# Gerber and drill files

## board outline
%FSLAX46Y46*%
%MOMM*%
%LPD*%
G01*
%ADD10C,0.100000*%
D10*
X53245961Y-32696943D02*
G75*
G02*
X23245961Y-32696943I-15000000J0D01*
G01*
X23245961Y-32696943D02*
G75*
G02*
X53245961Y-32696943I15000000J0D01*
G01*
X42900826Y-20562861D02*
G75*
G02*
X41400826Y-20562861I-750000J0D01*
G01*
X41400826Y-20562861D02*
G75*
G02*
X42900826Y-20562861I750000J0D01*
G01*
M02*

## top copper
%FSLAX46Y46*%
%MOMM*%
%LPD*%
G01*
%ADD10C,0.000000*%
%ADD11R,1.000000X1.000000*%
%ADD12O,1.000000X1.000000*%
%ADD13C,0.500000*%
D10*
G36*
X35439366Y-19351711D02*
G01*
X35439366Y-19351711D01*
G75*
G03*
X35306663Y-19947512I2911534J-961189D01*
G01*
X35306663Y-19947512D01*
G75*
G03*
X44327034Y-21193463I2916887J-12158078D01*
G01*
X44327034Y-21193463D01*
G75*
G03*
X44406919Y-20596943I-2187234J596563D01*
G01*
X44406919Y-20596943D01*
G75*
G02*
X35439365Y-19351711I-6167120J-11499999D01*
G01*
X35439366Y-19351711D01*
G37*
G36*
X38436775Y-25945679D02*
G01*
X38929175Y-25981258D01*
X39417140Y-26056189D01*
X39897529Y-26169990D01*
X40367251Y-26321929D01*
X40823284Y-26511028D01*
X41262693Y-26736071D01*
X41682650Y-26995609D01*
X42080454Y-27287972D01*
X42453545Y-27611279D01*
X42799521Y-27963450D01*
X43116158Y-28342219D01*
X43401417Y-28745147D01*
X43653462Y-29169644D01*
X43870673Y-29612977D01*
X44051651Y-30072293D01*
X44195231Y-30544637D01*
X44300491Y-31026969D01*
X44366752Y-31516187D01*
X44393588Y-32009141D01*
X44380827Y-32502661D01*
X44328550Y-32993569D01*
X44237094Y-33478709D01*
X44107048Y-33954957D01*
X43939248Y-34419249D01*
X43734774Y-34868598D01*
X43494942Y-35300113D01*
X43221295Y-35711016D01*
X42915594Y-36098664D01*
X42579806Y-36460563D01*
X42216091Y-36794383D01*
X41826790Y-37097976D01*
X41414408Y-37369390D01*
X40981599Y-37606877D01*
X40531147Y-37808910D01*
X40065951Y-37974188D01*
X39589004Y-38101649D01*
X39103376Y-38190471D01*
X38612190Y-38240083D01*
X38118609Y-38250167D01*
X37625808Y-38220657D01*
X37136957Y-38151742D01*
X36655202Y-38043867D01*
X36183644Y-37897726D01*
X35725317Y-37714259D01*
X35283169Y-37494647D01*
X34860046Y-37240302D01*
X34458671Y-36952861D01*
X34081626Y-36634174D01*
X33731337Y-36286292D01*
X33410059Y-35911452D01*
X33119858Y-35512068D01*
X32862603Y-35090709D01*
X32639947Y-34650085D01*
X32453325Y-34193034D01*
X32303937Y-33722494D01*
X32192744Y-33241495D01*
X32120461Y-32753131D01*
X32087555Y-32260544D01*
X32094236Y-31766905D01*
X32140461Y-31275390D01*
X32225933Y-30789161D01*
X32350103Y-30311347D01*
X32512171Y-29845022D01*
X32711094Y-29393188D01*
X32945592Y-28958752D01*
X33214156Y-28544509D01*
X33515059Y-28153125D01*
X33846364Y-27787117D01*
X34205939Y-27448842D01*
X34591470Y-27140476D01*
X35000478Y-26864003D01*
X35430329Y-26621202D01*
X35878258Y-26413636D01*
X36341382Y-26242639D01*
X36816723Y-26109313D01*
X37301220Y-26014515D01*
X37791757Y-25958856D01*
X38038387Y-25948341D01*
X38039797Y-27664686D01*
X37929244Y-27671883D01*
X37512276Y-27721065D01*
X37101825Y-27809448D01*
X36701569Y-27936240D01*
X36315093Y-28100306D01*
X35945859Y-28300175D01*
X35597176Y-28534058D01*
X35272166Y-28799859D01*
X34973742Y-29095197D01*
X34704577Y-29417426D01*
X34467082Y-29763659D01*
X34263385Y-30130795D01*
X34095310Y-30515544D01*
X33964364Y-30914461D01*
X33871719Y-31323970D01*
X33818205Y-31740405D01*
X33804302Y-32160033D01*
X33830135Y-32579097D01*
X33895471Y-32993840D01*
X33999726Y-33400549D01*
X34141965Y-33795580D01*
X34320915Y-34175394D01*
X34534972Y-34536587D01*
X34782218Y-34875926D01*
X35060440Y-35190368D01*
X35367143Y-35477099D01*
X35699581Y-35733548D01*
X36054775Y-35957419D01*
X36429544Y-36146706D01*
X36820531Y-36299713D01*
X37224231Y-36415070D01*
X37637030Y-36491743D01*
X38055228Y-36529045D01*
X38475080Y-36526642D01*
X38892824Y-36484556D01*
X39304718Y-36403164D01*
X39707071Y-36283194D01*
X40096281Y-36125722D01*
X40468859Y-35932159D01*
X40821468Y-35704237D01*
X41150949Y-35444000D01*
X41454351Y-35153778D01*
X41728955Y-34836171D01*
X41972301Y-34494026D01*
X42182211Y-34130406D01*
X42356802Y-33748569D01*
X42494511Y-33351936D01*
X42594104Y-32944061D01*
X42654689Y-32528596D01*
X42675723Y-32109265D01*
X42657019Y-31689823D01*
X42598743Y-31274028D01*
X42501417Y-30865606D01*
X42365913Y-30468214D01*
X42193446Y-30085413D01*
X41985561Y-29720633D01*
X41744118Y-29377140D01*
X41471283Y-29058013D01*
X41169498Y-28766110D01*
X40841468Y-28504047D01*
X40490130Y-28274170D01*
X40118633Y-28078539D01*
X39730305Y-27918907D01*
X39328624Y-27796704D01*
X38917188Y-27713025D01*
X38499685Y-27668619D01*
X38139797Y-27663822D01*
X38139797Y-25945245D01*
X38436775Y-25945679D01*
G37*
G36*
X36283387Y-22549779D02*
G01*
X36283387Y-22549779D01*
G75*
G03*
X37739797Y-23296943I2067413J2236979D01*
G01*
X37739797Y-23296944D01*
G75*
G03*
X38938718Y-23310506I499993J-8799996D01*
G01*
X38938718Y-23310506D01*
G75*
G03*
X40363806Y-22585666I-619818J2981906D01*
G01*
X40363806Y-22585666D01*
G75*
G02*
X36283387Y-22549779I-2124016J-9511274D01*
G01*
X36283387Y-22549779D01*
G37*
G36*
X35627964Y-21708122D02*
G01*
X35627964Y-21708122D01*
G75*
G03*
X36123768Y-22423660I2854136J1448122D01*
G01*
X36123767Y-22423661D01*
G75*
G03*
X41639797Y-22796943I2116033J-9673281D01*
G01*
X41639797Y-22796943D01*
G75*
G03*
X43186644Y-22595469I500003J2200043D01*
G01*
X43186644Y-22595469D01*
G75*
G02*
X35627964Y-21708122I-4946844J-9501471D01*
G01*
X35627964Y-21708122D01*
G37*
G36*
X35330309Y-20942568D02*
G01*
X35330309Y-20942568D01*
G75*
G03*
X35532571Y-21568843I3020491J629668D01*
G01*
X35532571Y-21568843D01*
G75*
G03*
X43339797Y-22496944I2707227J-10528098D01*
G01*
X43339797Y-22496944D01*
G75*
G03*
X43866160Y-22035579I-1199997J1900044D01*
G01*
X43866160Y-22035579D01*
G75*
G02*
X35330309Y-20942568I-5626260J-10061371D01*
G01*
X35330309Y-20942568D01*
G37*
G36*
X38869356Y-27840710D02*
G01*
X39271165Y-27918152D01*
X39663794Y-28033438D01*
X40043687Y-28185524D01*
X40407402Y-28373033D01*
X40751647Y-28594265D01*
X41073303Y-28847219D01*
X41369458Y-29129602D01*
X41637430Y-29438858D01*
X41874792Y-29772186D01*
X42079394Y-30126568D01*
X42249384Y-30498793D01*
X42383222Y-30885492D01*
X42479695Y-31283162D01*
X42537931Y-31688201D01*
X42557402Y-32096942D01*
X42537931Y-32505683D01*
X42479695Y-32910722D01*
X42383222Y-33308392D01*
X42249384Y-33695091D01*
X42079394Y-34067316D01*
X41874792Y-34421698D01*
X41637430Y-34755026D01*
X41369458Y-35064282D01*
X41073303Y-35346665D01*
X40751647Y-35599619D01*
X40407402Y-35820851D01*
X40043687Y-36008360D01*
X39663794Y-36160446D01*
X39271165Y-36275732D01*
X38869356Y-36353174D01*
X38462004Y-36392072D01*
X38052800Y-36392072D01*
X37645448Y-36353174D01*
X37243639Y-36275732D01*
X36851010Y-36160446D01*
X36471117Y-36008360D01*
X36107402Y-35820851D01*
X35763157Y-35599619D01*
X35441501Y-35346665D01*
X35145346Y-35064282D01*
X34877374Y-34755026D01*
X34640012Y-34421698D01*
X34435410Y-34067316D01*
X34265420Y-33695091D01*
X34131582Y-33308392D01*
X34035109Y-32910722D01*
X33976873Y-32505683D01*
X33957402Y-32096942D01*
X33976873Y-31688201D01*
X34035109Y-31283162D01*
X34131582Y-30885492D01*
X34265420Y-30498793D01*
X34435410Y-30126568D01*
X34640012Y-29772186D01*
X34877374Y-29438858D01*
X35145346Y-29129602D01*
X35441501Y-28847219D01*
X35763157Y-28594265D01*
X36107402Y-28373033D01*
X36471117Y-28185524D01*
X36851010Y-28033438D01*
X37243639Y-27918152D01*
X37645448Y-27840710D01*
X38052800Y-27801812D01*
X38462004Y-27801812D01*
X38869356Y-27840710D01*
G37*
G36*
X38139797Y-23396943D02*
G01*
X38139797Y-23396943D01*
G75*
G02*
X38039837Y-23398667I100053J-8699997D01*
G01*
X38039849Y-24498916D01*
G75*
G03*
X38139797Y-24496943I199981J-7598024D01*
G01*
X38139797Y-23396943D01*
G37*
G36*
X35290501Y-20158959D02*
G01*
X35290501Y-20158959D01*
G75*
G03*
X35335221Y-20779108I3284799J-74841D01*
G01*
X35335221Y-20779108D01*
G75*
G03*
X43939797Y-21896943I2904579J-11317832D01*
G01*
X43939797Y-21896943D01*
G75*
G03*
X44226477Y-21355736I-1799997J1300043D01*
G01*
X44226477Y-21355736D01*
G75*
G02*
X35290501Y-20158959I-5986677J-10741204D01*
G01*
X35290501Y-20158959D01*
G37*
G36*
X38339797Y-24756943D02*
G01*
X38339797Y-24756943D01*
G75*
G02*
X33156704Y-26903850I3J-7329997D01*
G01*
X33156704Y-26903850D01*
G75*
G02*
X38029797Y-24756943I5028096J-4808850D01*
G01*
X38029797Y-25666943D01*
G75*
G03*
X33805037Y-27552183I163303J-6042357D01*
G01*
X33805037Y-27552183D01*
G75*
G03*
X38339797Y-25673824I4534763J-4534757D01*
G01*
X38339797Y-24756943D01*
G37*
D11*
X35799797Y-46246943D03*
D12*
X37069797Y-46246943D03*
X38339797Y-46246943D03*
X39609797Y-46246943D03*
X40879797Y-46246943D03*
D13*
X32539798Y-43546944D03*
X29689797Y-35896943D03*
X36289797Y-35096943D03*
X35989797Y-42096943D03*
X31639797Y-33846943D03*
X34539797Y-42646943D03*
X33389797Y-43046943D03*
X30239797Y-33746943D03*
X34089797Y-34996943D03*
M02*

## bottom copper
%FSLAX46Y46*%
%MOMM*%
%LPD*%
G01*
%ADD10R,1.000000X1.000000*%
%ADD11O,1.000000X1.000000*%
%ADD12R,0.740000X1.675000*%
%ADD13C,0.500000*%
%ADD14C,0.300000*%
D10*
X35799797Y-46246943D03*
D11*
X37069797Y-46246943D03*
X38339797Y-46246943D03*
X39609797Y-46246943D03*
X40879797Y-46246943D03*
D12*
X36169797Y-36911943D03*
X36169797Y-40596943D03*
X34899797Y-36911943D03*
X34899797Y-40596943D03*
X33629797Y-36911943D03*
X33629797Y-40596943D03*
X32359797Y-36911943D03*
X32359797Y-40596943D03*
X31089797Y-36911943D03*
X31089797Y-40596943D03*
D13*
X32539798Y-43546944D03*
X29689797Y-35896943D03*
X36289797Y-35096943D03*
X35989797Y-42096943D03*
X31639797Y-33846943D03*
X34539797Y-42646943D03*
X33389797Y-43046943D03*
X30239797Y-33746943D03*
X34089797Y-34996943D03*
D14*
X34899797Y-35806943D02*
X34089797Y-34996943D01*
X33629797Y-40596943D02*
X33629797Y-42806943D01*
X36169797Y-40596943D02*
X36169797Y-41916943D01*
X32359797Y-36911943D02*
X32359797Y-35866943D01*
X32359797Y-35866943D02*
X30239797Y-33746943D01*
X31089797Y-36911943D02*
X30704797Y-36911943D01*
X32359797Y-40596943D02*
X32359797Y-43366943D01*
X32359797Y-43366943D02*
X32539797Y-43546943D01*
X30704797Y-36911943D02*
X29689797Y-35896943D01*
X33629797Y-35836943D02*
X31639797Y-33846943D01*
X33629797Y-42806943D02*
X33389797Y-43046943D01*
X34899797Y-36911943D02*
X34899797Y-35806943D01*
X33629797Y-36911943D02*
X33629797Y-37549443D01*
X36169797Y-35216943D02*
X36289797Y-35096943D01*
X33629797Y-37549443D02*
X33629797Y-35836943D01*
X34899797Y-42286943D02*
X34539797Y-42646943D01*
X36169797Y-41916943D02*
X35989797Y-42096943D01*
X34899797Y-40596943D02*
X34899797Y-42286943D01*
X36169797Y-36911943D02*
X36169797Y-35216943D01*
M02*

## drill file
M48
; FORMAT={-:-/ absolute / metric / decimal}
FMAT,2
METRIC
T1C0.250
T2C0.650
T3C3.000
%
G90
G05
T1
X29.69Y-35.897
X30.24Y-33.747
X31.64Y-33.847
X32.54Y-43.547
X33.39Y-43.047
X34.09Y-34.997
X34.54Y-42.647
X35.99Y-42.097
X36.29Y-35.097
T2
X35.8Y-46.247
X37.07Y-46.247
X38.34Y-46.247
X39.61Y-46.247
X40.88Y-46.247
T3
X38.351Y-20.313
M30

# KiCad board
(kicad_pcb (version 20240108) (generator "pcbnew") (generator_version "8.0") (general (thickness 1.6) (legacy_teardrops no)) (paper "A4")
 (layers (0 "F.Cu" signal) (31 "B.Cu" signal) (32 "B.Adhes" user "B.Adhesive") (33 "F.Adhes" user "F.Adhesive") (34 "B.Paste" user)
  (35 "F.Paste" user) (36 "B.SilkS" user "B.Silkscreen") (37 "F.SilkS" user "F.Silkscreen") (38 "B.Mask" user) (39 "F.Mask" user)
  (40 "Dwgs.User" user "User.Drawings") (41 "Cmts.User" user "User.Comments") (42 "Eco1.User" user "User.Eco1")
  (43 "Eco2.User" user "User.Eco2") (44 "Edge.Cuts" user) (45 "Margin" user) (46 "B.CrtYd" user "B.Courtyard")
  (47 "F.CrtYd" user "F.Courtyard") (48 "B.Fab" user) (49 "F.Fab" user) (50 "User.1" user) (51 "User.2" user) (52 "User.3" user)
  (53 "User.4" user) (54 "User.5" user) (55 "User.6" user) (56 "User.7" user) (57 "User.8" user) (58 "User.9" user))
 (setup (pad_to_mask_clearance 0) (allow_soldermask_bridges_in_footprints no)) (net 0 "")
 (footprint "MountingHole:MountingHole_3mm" (layer "F.Cu") (at 38.350826 20.312861)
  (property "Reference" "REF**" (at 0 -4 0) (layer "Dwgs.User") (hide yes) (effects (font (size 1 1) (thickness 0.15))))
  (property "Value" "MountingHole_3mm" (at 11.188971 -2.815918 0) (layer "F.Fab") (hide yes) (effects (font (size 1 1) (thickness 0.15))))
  (pad "" np_thru_hole circle (at 0 0) (size 3 3) (drill 3) (layers "*.Cu" "*.Mask")))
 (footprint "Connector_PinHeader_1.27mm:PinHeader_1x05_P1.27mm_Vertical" (layer "F.Cu") (at 35.799797 46.246943 90)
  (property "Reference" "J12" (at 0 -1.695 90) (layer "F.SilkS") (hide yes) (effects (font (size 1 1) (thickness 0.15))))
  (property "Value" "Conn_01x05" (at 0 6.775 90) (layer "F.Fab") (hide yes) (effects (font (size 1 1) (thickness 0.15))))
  (pad "1" thru_hole rect (at 0 0 90) (size 1 1) (drill 0.65) (layers "*.Cu" "*.Mask") (remove_unused_layers no))
  (pad "2" thru_hole oval (at 0 1.27 90) (size 1 1) (drill 0.65) (layers "*.Cu" "*.Mask") (remove_unused_layers no))
  (pad "3" thru_hole oval (at 0 2.54 90) (size 1 1) (drill 0.65) (layers "*.Cu" "*.Mask") (remove_unused_layers no))
  (pad "4" thru_hole oval (at 0 3.81 90) (size 1 1) (drill 0.65) (layers "*.Cu" "*.Mask") (remove_unused_layers no))
  (pad "5" thru_hole oval (at 0 5.08 90) (size 1 1) (drill 0.65) (layers "*.Cu" "*.Mask") (remove_unused_layers no)))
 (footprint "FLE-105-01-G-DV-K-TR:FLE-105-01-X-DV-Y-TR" (layer "B.Cu") (at 33.629797 38.754443 180)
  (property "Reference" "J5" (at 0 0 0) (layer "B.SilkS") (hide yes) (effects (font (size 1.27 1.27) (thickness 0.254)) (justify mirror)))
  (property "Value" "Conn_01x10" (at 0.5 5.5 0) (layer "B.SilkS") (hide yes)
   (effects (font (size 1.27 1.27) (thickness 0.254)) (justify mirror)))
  (pad "1" smd rect (at -2.54 1.8425 180) (size 0.74 1.675) (layers "B.Cu" "B.Paste" "B.Mask"))
  (pad "2" smd rect (at -2.54 -1.8425 180) (size 0.74 1.675) (layers "B.Cu" "B.Paste" "B.Mask"))
  (pad "3" smd rect (at -1.27 1.8425 180) (size 0.74 1.675) (layers "B.Cu" "B.Paste" "B.Mask"))
  (pad "4" smd rect (at -1.27 -1.8425 180) (size 0.74 1.675) (layers "B.Cu" "B.Paste" "B.Mask"))
  (pad "5" smd rect (at 0 1.8425 180) (size 0.74 1.675) (layers "B.Cu" "B.Paste" "B.Mask"))
  (pad "6" smd rect (at 0 -1.8425 180) (size 0.74 1.675) (layers "B.Cu" "B.Paste" "B.Mask"))
  (pad "7" smd rect (at 1.27 1.8425 180) (size 0.74 1.675) (layers "B.Cu" "B.Paste" "B.Mask"))
  (pad "8" smd rect (at 1.27 -1.8425 180) (size 0.74 1.675) (layers "B.Cu" "B.Paste" "B.Mask"))
  (pad "9" smd rect (at 2.54 1.8425 180) (size 0.74 1.675) (layers "B.Cu" "B.Paste" "B.Mask"))
  (pad "10" smd rect (at 2.54 -1.8425 180) (size 0.74 1.675) (layers "B.Cu" "B.Paste" "B.Mask")))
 (gr_poly
  (pts
   (arc (start 35.439365 19.351711) (mid 36.445003 45.022191) (end 44.406919 20.596943))
   (arc (start 44.406919 20.596943) (mid 44.386859 20.897866) (end 44.327034 21.193463))
   (arc (start 44.327034 21.193463) (mid 36.512783 44.491082) (end 35.306663 19.947512))
   (arc (start 35.306663 19.947512) (mid 35.358151 19.646301) (end 35.439366 19.351711)))
  (stroke (width 0) (type solid)) (fill solid) (layer "F.Cu"))
 (gr_poly
  (pts (xy 38.139797 25.945245) (xy 38.436775 25.945679) (xy 38.929175 25.981258) (xy 39.41714 26.056189) (xy 39.897529 26.16999)
   (xy 40.367251 26.321929) (xy 40.823284 26.511028) (xy 41.262693 26.736071) (xy 41.68265 26.995609) (xy 42.080454 27.287972)
   (xy 42.453545 27.611279) (xy 42.799521 27.96345) (xy 43.116158 28.342219) (xy 43.401417 28.745147) (xy 43.653462 29.169644)
   (xy 43.870673 29.612977) (xy 44.051651 30.072293) (xy 44.195231 30.544637) (xy 44.300491 31.026969) (xy 44.366752 31.516187)
   (xy 44.393588 32.009141) (xy 44.380827 32.502661) (xy 44.32855 32.993569) (xy 44.237094 33.478709) (xy 44.107048 33.954957)
   (xy 43.939248 34.419249) (xy 43.734774 34.868598) (xy 43.494942 35.300113) (xy 43.221295 35.711016) (xy 42.915594 36.098664)
   (xy 42.579806 36.460563) (xy 42.216091 36.794383) (xy 41.82679 37.097976) (xy 41.414408 37.36939) (xy 40.981599 37.606877)
   (xy 40.531147 37.80891) (xy 40.065951 37.974188) (xy 39.589004 38.101649) (xy 39.103376 38.190471) (xy 38.61219 38.240083)
   (xy 38.118609 38.250167) (xy 37.625808 38.220657) (xy 37.136957 38.151742) (xy 36.655202 38.043867) (xy 36.183644 37.897726)
   (xy 35.725317 37.714259) (xy 35.283169 37.494647) (xy 34.860046 37.240302) (xy 34.458671 36.952861) (xy 34.081626 36.634174)
   (xy 33.731337 36.286292) (xy 33.410059 35.911452) (xy 33.119858 35.512068) (xy 32.862603 35.090709) (xy 32.639947 34.650085)
   (xy 32.453325 34.193034) (xy 32.303937 33.722494) (xy 32.192744 33.241495) (xy 32.120461 32.753131) (xy 32.087555 32.260544)
   (xy 32.094236 31.766905) (xy 32.140461 31.27539) (xy 32.225933 30.789161) (xy 32.350103 30.311347) (xy 32.512171 29.845022)
   (xy 32.711094 29.393188) (xy 32.945592 28.958752) (xy 33.214156 28.544509) (xy 33.515059 28.153125) (xy 33.846364 27.787117)
   (xy 34.205939 27.448842) (xy 34.59147 27.140476) (xy 35.000478 26.864003) (xy 35.430329 26.621202) (xy 35.878258 26.413636)
   (xy 36.341382 26.242639) (xy 36.816723 26.109313) (xy 37.30122 26.014515) (xy 37.791757 25.958856) (xy 38.038387 25.948341)
   (xy 38.039797 27.664686) (xy 37.929244 27.671883) (xy 37.512276 27.721065) (xy 37.101825 27.809448) (xy 36.701569 27.93624)
   (xy 36.315093 28.100306) (xy 35.945859 28.300175) (xy 35.597176 28.534058) (xy 35.272166 28.799859) (xy 34.973742 29.095197)
   (xy 34.704577 29.417426) (xy 34.467082 29.763659) (xy 34.263385 30.130795) (xy 34.09531 30.515544) (xy 33.964364 30.914461)
   (xy 33.871719 31.32397) (xy 33.818205 31.740405) (xy 33.804302 32.160033) (xy 33.830135 32.579097) (xy 33.895471 32.99384)
   (xy 33.999726 33.400549) (xy 34.141965 33.79558) (xy 34.320915 34.175394) (xy 34.534972 34.536587) (xy 34.782218 34.875926)
   (xy 35.06044 35.190368) (xy 35.367143 35.477099) (xy 35.699581 35.733548) (xy 36.054775 35.957419) (xy 36.429544 36.146706)
   (xy 36.820531 36.299713) (xy 37.224231 36.41507) (xy 37.63703 36.491743) (xy 38.055228 36.529045) (xy 38.47508 36.526642)
   (xy 38.892824 36.484556) (xy 39.304718 36.403164) (xy 39.707071 36.283194) (xy 40.096281 36.125722) (xy 40.468859 35.932159)
   (xy 40.821468 35.704237) (xy 41.150949 35.444) (xy 41.454351 35.153778) (xy 41.728955 34.836171) (xy 41.972301 34.494026)
   (xy 42.182211 34.130406) (xy 42.356802 33.748569) (xy 42.494511 33.351936) (xy 42.594104 32.944061) (xy 42.654689 32.528596)
   (xy 42.675723 32.109265) (xy 42.657019 31.689823) (xy 42.598743 31.274028) (xy 42.501417 30.865606) (xy 42.365913 30.468214)
   (xy 42.193446 30.085413) (xy 41.985561 29.720633) (xy 41.744118 29.37714) (xy 41.471283 29.058013) (xy 41.169498 28.76611)
   (xy 40.841468 28.504047) (xy 40.49013 28.27417) (xy 40.118633 28.078539) (xy 39.730305 27.918907) (xy 39.328624 27.796704)
   (xy 38.917188 27.713025) (xy 38.499685 27.668619) (xy 38.139797 27.663822))
  (stroke (width 0) (type solid)) (fill solid) (layer "F.Cu"))
 (gr_poly
  (pts
   (arc (start 37.739797 23.296944) (mid 38.140092 40.910567) (end 38.938718 23.310506))
   (arc (start 38.938718 23.310506) (mid 39.699675 23.04327) (end 40.363806 22.585666))
   (arc (start 40.363806 22.585666) (mid 38.154082 41.842117) (end 36.283387 22.549779))
   (arc (start 36.283387 22.549779) (mid 36.960462 23.023025) (end 37.739797 23.296943)))
  (stroke (width 0) (type solid)) (fill solid) (layer "F.Cu"))
 (gr_poly
  (pts
   (arc (start 36.123767 22.423661) (mid 37.571236 41.976365) (end 41.639797 22.796943))
   (arc (start 41.639797 22.796943) (mid 42.431187 22.834148) (end 43.186644 22.595469))
   (arc (start 43.186644 22.595469) (mid 36.990834 42.73599) (end 35.627964 21.708122))
   (arc (start 35.627964 21.708122) (mid 35.851424 22.082827) (end 36.123768 22.42366)))
  (stroke (width 0) (type solid)) (fill solid) (layer "F.Cu"))
 (gr_poly
  (pts
   (arc (start 43.339797 22.496944) (mid 43.621051 22.28688) (end 43.86616 22.035579))
   (arc (start 43.86616 22.035579) (mid 36.77575 43.531215) (end 35.330309 20.942568))
   (arc (start 35.330309 20.942568) (mid 35.414694 21.261114) (end 35.532571 21.568843))
   (arc (start 35.532571 21.568843) (mid 36.956567 42.891535) (end 43.339797 22.496944)))
  (stroke (width 0) (type solid)) (fill solid) (layer "F.Cu"))
 (gr_poly
  (pts (xy 42.557402 32.096942) (xy 42.537931 31.688201) (xy 42.479695 31.283162) (xy 42.383222 30.885492) (xy 42.249384 30.498793)
   (xy 42.079394 30.126568) (xy 41.874792 29.772186) (xy 41.63743 29.438858) (xy 41.369458 29.129602) (xy 41.073303 28.847219)
   (xy 40.751647 28.594265) (xy 40.407402 28.373033) (xy 40.043687 28.185524) (xy 39.663794 28.033438) (xy 39.271165 27.918152)
   (xy 38.869356 27.84071) (xy 38.462004 27.801812) (xy 38.0528 27.801812) (xy 37.645448 27.84071) (xy 37.243639 27.918152)
   (xy 36.85101 28.033438) (xy 36.471117 28.185524) (xy 36.107402 28.373033) (xy 35.763157 28.594265) (xy 35.441501 28.847219)
   (xy 35.145346 29.129602) (xy 34.877374 29.438858) (xy 34.640012 29.772186) (xy 34.43541 30.126568) (xy 34.26542 30.498793)
   (xy 34.131582 30.885492) (xy 34.035109 31.283162) (xy 33.976873 31.688201) (xy 33.957402 32.096942) (xy 33.976873 32.505683)
   (xy 34.035109 32.910722) (xy 34.131582 33.308392) (xy 34.26542 33.695091) (xy 34.43541 34.067316) (xy 34.640012 34.421698)
   (xy 34.877374 34.755026) (xy 35.145346 35.064282) (xy 35.441501 35.346665) (xy 35.763157 35.599619) (xy 36.107402 35.820851)
   (xy 36.471117 36.00836) (xy 36.85101 36.160446) (xy 37.243639 36.275732) (xy 37.645448 36.353174) (xy 38.0528 36.392072)
   (xy 38.462004 36.392072) (xy 38.869356 36.353174) (xy 39.271165 36.275732) (xy 39.663794 36.160446) (xy 40.043687 36.00836)
   (xy 40.407402 35.820851) (xy 40.751647 35.599619) (xy 41.073303 35.346665) (xy 41.369458 35.064282) (xy 41.63743 34.755026)
   (xy 41.874792 34.421698) (xy 42.079394 34.067316) (xy 42.249384 33.695091) (xy 42.383222 33.308392) (xy 42.479695 32.910722)
   (xy 42.537931 32.505683) (xy 42.557402 32.096942))
  (stroke (width 0) (type solid)) (fill solid) (layer "F.Cu"))
 (gr_poly
  (pts
   (arc (start 38.039849 24.498916) (mid 38.389838 39.696115) (end 38.139797 24.496943))
   (arc (start 38.139797 23.396943) (mid 38.389885 40.796217) (end 38.039837 23.398667)))
  (stroke (width 0) (type solid)) (fill solid) (layer "F.Cu"))
 (gr_poly
  (pts
   (arc (start 35.335221 20.779108) (mid 36.734483 43.684171) (end 43.939797 21.896943))
   (arc (start 43.939797 21.896943) (mid 44.101887 21.636271) (end 44.226477 21.355736))
   (arc (start 44.226477 21.355736) (mid 36.607475 44.285021) (end 35.290501 20.158959))
   (arc (start 35.290501 20.158959) (mid 35.298159 20.470094) (end 35.335221 20.779108)))
  (stroke (width 0) (type solid)) (fill solid) (layer "F.Cu"))
 (gr_poly
  (pts
   (arc (start 33.156704 26.90385) (mid 41.144867 38.85898) (end 38.339797 24.756943))
   (arc (start 38.339797 25.673824) (mid 40.793991 38.011892) (end 33.805037 27.552183))
   (arc (start 33.805037 27.552183) (mid 35.729918 26.189385) (end 38.029797 25.666943))
   (arc (start 38.029797 24.756943) (mid 35.379727 25.345737) (end 33.156704 26.90385)))
  (stroke (width 0) (type solid)) (fill solid) (layer "F.Cu"))
 (gr_circle (center 38.245961 32.696943) (end 53.245961 32.696943) (stroke (width 0.1) (type default)) (fill none) (layer "Edge.Cuts"))
 (gr_circle (center 42.150826 20.562861) (end 42.900826 20.562861) (stroke (width 0.1) (type default)) (fill none) (layer "Edge.Cuts"))
 (via (at 32.539798 43.546944) (size 0.5) (drill 0.25) (layers "F.Cu" "B.Cu") (remove_unused_layers yes) (keep_end_layers yes)
  (zone_layer_connections) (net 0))
 (via (at 29.689797 35.896943) (size 0.5) (drill 0.25) (layers "F.Cu" "B.Cu") (remove_unused_layers yes) (keep_end_layers yes)
  (zone_layer_connections) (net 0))
 (via (at 36.289797 35.096943) (size 0.5) (drill 0.25) (layers "F.Cu" "B.Cu") (remove_unused_layers yes) (keep_end_layers yes)
  (zone_layer_connections) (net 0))
 (via (at 35.989797 42.096943) (size 0.5) (drill 0.25) (layers "F.Cu" "B.Cu") (remove_unused_layers yes) (keep_end_layers yes)
  (zone_layer_connections) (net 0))
 (via (at 31.639797 33.846943) (size 0.5) (drill 0.25) (layers "F.Cu" "B.Cu") (remove_unused_layers yes) (keep_end_layers yes)
  (zone_layer_connections) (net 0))
 (via (at 34.539797 42.646943) (size 0.5) (drill 0.25) (layers "F.Cu" "B.Cu") (remove_unused_layers yes) (keep_end_layers yes)
  (zone_layer_connections) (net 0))
 (via (at 33.389797 43.046943) (size 0.5) (drill 0.25) (layers "F.Cu" "B.Cu") (remove_unused_layers yes) (keep_end_layers yes)
  (zone_layer_connections) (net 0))
 (via (at 30.239797 33.746943) (size 0.5) (drill 0.25) (layers "F.Cu" "B.Cu") (remove_unused_layers yes) (keep_end_layers yes)
  (zone_layer_connections) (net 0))
 (via (at 34.089797 34.996943) (size 0.5) (drill 0.25) (layers "F.Cu" "B.Cu") (remove_unused_layers yes) (keep_end_layers yes)
  (zone_layer_connections) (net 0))
 (segment (start 34.899797 35.806943) (end 34.089797 34.996943) (width 0.3) (layer "B.Cu") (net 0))
 (segment (start 33.629797 40.596943) (end 33.629797 42.806943) (width 0.3) (layer "B.Cu") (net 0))
 (segment (start 36.169797 40.596943) (end 36.169797 41.916943) (width 0.3) (layer "B.Cu") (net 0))
 (segment (start 32.359797 36.911943) (end 32.359797 35.866943) (width 0.3) (layer "B.Cu") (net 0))
 (segment (start 32.359797 35.866943) (end 30.239797 33.746943) (width 0.3) (layer "B.Cu") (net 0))
 (segment (start 31.089797 36.911943) (end 30.704797 36.911943) (width 0.3) (layer "B.Cu") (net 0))
 (segment (start 32.359797 40.596943) (end 32.359797 43.366943) (width 0.3) (layer "B.Cu") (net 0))
 (segment (start 32.359797 43.366943) (end 32.539797 43.546943) (width 0.3) (layer "B.Cu") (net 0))
 (segment (start 30.704797 36.911943) (end 29.689797 35.896943) (width 0.3) (layer "B.Cu") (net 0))
 (segment (start 33.629797 35.836943) (end 31.639797 33.846943) (width 0.3) (layer "B.Cu") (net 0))
 (segment (start 33.629797 42.806943) (end 33.389797 43.046943) (width 0.3) (layer "B.Cu") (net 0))
 (segment (start 34.899797 36.911943) (end 34.899797 35.806943) (width 0.3) (layer "B.Cu") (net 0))
 (segment (start 33.629797 36.911943) (end 33.629797 37.549443) (width 0.3) (layer "B.Cu") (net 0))
 (segment (start 36.169797 35.216943) (end 36.289797 35.096943) (width 0.3) (layer "B.Cu") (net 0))
 (segment (start 33.629797 37.549443) (end 33.629797 35.836943) (width 0.3) (layer "B.Cu") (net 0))
 (segment (start 34.899797 42.286943) (end 34.539797 42.646943) (width 0.3) (layer "B.Cu") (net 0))
 (segment (start 36.169797 41.916943) (end 35.989797 42.096943) (width 0.3) (layer "B.Cu") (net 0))
 (segment (start 34.899797 40.596943) (end 34.899797 42.286943) (width 0.3) (layer "B.Cu") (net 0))
 (segment (start 36.169797 36.911943) (end 36.169797 35.216943) (width 0.3) (layer "B.Cu") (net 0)))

